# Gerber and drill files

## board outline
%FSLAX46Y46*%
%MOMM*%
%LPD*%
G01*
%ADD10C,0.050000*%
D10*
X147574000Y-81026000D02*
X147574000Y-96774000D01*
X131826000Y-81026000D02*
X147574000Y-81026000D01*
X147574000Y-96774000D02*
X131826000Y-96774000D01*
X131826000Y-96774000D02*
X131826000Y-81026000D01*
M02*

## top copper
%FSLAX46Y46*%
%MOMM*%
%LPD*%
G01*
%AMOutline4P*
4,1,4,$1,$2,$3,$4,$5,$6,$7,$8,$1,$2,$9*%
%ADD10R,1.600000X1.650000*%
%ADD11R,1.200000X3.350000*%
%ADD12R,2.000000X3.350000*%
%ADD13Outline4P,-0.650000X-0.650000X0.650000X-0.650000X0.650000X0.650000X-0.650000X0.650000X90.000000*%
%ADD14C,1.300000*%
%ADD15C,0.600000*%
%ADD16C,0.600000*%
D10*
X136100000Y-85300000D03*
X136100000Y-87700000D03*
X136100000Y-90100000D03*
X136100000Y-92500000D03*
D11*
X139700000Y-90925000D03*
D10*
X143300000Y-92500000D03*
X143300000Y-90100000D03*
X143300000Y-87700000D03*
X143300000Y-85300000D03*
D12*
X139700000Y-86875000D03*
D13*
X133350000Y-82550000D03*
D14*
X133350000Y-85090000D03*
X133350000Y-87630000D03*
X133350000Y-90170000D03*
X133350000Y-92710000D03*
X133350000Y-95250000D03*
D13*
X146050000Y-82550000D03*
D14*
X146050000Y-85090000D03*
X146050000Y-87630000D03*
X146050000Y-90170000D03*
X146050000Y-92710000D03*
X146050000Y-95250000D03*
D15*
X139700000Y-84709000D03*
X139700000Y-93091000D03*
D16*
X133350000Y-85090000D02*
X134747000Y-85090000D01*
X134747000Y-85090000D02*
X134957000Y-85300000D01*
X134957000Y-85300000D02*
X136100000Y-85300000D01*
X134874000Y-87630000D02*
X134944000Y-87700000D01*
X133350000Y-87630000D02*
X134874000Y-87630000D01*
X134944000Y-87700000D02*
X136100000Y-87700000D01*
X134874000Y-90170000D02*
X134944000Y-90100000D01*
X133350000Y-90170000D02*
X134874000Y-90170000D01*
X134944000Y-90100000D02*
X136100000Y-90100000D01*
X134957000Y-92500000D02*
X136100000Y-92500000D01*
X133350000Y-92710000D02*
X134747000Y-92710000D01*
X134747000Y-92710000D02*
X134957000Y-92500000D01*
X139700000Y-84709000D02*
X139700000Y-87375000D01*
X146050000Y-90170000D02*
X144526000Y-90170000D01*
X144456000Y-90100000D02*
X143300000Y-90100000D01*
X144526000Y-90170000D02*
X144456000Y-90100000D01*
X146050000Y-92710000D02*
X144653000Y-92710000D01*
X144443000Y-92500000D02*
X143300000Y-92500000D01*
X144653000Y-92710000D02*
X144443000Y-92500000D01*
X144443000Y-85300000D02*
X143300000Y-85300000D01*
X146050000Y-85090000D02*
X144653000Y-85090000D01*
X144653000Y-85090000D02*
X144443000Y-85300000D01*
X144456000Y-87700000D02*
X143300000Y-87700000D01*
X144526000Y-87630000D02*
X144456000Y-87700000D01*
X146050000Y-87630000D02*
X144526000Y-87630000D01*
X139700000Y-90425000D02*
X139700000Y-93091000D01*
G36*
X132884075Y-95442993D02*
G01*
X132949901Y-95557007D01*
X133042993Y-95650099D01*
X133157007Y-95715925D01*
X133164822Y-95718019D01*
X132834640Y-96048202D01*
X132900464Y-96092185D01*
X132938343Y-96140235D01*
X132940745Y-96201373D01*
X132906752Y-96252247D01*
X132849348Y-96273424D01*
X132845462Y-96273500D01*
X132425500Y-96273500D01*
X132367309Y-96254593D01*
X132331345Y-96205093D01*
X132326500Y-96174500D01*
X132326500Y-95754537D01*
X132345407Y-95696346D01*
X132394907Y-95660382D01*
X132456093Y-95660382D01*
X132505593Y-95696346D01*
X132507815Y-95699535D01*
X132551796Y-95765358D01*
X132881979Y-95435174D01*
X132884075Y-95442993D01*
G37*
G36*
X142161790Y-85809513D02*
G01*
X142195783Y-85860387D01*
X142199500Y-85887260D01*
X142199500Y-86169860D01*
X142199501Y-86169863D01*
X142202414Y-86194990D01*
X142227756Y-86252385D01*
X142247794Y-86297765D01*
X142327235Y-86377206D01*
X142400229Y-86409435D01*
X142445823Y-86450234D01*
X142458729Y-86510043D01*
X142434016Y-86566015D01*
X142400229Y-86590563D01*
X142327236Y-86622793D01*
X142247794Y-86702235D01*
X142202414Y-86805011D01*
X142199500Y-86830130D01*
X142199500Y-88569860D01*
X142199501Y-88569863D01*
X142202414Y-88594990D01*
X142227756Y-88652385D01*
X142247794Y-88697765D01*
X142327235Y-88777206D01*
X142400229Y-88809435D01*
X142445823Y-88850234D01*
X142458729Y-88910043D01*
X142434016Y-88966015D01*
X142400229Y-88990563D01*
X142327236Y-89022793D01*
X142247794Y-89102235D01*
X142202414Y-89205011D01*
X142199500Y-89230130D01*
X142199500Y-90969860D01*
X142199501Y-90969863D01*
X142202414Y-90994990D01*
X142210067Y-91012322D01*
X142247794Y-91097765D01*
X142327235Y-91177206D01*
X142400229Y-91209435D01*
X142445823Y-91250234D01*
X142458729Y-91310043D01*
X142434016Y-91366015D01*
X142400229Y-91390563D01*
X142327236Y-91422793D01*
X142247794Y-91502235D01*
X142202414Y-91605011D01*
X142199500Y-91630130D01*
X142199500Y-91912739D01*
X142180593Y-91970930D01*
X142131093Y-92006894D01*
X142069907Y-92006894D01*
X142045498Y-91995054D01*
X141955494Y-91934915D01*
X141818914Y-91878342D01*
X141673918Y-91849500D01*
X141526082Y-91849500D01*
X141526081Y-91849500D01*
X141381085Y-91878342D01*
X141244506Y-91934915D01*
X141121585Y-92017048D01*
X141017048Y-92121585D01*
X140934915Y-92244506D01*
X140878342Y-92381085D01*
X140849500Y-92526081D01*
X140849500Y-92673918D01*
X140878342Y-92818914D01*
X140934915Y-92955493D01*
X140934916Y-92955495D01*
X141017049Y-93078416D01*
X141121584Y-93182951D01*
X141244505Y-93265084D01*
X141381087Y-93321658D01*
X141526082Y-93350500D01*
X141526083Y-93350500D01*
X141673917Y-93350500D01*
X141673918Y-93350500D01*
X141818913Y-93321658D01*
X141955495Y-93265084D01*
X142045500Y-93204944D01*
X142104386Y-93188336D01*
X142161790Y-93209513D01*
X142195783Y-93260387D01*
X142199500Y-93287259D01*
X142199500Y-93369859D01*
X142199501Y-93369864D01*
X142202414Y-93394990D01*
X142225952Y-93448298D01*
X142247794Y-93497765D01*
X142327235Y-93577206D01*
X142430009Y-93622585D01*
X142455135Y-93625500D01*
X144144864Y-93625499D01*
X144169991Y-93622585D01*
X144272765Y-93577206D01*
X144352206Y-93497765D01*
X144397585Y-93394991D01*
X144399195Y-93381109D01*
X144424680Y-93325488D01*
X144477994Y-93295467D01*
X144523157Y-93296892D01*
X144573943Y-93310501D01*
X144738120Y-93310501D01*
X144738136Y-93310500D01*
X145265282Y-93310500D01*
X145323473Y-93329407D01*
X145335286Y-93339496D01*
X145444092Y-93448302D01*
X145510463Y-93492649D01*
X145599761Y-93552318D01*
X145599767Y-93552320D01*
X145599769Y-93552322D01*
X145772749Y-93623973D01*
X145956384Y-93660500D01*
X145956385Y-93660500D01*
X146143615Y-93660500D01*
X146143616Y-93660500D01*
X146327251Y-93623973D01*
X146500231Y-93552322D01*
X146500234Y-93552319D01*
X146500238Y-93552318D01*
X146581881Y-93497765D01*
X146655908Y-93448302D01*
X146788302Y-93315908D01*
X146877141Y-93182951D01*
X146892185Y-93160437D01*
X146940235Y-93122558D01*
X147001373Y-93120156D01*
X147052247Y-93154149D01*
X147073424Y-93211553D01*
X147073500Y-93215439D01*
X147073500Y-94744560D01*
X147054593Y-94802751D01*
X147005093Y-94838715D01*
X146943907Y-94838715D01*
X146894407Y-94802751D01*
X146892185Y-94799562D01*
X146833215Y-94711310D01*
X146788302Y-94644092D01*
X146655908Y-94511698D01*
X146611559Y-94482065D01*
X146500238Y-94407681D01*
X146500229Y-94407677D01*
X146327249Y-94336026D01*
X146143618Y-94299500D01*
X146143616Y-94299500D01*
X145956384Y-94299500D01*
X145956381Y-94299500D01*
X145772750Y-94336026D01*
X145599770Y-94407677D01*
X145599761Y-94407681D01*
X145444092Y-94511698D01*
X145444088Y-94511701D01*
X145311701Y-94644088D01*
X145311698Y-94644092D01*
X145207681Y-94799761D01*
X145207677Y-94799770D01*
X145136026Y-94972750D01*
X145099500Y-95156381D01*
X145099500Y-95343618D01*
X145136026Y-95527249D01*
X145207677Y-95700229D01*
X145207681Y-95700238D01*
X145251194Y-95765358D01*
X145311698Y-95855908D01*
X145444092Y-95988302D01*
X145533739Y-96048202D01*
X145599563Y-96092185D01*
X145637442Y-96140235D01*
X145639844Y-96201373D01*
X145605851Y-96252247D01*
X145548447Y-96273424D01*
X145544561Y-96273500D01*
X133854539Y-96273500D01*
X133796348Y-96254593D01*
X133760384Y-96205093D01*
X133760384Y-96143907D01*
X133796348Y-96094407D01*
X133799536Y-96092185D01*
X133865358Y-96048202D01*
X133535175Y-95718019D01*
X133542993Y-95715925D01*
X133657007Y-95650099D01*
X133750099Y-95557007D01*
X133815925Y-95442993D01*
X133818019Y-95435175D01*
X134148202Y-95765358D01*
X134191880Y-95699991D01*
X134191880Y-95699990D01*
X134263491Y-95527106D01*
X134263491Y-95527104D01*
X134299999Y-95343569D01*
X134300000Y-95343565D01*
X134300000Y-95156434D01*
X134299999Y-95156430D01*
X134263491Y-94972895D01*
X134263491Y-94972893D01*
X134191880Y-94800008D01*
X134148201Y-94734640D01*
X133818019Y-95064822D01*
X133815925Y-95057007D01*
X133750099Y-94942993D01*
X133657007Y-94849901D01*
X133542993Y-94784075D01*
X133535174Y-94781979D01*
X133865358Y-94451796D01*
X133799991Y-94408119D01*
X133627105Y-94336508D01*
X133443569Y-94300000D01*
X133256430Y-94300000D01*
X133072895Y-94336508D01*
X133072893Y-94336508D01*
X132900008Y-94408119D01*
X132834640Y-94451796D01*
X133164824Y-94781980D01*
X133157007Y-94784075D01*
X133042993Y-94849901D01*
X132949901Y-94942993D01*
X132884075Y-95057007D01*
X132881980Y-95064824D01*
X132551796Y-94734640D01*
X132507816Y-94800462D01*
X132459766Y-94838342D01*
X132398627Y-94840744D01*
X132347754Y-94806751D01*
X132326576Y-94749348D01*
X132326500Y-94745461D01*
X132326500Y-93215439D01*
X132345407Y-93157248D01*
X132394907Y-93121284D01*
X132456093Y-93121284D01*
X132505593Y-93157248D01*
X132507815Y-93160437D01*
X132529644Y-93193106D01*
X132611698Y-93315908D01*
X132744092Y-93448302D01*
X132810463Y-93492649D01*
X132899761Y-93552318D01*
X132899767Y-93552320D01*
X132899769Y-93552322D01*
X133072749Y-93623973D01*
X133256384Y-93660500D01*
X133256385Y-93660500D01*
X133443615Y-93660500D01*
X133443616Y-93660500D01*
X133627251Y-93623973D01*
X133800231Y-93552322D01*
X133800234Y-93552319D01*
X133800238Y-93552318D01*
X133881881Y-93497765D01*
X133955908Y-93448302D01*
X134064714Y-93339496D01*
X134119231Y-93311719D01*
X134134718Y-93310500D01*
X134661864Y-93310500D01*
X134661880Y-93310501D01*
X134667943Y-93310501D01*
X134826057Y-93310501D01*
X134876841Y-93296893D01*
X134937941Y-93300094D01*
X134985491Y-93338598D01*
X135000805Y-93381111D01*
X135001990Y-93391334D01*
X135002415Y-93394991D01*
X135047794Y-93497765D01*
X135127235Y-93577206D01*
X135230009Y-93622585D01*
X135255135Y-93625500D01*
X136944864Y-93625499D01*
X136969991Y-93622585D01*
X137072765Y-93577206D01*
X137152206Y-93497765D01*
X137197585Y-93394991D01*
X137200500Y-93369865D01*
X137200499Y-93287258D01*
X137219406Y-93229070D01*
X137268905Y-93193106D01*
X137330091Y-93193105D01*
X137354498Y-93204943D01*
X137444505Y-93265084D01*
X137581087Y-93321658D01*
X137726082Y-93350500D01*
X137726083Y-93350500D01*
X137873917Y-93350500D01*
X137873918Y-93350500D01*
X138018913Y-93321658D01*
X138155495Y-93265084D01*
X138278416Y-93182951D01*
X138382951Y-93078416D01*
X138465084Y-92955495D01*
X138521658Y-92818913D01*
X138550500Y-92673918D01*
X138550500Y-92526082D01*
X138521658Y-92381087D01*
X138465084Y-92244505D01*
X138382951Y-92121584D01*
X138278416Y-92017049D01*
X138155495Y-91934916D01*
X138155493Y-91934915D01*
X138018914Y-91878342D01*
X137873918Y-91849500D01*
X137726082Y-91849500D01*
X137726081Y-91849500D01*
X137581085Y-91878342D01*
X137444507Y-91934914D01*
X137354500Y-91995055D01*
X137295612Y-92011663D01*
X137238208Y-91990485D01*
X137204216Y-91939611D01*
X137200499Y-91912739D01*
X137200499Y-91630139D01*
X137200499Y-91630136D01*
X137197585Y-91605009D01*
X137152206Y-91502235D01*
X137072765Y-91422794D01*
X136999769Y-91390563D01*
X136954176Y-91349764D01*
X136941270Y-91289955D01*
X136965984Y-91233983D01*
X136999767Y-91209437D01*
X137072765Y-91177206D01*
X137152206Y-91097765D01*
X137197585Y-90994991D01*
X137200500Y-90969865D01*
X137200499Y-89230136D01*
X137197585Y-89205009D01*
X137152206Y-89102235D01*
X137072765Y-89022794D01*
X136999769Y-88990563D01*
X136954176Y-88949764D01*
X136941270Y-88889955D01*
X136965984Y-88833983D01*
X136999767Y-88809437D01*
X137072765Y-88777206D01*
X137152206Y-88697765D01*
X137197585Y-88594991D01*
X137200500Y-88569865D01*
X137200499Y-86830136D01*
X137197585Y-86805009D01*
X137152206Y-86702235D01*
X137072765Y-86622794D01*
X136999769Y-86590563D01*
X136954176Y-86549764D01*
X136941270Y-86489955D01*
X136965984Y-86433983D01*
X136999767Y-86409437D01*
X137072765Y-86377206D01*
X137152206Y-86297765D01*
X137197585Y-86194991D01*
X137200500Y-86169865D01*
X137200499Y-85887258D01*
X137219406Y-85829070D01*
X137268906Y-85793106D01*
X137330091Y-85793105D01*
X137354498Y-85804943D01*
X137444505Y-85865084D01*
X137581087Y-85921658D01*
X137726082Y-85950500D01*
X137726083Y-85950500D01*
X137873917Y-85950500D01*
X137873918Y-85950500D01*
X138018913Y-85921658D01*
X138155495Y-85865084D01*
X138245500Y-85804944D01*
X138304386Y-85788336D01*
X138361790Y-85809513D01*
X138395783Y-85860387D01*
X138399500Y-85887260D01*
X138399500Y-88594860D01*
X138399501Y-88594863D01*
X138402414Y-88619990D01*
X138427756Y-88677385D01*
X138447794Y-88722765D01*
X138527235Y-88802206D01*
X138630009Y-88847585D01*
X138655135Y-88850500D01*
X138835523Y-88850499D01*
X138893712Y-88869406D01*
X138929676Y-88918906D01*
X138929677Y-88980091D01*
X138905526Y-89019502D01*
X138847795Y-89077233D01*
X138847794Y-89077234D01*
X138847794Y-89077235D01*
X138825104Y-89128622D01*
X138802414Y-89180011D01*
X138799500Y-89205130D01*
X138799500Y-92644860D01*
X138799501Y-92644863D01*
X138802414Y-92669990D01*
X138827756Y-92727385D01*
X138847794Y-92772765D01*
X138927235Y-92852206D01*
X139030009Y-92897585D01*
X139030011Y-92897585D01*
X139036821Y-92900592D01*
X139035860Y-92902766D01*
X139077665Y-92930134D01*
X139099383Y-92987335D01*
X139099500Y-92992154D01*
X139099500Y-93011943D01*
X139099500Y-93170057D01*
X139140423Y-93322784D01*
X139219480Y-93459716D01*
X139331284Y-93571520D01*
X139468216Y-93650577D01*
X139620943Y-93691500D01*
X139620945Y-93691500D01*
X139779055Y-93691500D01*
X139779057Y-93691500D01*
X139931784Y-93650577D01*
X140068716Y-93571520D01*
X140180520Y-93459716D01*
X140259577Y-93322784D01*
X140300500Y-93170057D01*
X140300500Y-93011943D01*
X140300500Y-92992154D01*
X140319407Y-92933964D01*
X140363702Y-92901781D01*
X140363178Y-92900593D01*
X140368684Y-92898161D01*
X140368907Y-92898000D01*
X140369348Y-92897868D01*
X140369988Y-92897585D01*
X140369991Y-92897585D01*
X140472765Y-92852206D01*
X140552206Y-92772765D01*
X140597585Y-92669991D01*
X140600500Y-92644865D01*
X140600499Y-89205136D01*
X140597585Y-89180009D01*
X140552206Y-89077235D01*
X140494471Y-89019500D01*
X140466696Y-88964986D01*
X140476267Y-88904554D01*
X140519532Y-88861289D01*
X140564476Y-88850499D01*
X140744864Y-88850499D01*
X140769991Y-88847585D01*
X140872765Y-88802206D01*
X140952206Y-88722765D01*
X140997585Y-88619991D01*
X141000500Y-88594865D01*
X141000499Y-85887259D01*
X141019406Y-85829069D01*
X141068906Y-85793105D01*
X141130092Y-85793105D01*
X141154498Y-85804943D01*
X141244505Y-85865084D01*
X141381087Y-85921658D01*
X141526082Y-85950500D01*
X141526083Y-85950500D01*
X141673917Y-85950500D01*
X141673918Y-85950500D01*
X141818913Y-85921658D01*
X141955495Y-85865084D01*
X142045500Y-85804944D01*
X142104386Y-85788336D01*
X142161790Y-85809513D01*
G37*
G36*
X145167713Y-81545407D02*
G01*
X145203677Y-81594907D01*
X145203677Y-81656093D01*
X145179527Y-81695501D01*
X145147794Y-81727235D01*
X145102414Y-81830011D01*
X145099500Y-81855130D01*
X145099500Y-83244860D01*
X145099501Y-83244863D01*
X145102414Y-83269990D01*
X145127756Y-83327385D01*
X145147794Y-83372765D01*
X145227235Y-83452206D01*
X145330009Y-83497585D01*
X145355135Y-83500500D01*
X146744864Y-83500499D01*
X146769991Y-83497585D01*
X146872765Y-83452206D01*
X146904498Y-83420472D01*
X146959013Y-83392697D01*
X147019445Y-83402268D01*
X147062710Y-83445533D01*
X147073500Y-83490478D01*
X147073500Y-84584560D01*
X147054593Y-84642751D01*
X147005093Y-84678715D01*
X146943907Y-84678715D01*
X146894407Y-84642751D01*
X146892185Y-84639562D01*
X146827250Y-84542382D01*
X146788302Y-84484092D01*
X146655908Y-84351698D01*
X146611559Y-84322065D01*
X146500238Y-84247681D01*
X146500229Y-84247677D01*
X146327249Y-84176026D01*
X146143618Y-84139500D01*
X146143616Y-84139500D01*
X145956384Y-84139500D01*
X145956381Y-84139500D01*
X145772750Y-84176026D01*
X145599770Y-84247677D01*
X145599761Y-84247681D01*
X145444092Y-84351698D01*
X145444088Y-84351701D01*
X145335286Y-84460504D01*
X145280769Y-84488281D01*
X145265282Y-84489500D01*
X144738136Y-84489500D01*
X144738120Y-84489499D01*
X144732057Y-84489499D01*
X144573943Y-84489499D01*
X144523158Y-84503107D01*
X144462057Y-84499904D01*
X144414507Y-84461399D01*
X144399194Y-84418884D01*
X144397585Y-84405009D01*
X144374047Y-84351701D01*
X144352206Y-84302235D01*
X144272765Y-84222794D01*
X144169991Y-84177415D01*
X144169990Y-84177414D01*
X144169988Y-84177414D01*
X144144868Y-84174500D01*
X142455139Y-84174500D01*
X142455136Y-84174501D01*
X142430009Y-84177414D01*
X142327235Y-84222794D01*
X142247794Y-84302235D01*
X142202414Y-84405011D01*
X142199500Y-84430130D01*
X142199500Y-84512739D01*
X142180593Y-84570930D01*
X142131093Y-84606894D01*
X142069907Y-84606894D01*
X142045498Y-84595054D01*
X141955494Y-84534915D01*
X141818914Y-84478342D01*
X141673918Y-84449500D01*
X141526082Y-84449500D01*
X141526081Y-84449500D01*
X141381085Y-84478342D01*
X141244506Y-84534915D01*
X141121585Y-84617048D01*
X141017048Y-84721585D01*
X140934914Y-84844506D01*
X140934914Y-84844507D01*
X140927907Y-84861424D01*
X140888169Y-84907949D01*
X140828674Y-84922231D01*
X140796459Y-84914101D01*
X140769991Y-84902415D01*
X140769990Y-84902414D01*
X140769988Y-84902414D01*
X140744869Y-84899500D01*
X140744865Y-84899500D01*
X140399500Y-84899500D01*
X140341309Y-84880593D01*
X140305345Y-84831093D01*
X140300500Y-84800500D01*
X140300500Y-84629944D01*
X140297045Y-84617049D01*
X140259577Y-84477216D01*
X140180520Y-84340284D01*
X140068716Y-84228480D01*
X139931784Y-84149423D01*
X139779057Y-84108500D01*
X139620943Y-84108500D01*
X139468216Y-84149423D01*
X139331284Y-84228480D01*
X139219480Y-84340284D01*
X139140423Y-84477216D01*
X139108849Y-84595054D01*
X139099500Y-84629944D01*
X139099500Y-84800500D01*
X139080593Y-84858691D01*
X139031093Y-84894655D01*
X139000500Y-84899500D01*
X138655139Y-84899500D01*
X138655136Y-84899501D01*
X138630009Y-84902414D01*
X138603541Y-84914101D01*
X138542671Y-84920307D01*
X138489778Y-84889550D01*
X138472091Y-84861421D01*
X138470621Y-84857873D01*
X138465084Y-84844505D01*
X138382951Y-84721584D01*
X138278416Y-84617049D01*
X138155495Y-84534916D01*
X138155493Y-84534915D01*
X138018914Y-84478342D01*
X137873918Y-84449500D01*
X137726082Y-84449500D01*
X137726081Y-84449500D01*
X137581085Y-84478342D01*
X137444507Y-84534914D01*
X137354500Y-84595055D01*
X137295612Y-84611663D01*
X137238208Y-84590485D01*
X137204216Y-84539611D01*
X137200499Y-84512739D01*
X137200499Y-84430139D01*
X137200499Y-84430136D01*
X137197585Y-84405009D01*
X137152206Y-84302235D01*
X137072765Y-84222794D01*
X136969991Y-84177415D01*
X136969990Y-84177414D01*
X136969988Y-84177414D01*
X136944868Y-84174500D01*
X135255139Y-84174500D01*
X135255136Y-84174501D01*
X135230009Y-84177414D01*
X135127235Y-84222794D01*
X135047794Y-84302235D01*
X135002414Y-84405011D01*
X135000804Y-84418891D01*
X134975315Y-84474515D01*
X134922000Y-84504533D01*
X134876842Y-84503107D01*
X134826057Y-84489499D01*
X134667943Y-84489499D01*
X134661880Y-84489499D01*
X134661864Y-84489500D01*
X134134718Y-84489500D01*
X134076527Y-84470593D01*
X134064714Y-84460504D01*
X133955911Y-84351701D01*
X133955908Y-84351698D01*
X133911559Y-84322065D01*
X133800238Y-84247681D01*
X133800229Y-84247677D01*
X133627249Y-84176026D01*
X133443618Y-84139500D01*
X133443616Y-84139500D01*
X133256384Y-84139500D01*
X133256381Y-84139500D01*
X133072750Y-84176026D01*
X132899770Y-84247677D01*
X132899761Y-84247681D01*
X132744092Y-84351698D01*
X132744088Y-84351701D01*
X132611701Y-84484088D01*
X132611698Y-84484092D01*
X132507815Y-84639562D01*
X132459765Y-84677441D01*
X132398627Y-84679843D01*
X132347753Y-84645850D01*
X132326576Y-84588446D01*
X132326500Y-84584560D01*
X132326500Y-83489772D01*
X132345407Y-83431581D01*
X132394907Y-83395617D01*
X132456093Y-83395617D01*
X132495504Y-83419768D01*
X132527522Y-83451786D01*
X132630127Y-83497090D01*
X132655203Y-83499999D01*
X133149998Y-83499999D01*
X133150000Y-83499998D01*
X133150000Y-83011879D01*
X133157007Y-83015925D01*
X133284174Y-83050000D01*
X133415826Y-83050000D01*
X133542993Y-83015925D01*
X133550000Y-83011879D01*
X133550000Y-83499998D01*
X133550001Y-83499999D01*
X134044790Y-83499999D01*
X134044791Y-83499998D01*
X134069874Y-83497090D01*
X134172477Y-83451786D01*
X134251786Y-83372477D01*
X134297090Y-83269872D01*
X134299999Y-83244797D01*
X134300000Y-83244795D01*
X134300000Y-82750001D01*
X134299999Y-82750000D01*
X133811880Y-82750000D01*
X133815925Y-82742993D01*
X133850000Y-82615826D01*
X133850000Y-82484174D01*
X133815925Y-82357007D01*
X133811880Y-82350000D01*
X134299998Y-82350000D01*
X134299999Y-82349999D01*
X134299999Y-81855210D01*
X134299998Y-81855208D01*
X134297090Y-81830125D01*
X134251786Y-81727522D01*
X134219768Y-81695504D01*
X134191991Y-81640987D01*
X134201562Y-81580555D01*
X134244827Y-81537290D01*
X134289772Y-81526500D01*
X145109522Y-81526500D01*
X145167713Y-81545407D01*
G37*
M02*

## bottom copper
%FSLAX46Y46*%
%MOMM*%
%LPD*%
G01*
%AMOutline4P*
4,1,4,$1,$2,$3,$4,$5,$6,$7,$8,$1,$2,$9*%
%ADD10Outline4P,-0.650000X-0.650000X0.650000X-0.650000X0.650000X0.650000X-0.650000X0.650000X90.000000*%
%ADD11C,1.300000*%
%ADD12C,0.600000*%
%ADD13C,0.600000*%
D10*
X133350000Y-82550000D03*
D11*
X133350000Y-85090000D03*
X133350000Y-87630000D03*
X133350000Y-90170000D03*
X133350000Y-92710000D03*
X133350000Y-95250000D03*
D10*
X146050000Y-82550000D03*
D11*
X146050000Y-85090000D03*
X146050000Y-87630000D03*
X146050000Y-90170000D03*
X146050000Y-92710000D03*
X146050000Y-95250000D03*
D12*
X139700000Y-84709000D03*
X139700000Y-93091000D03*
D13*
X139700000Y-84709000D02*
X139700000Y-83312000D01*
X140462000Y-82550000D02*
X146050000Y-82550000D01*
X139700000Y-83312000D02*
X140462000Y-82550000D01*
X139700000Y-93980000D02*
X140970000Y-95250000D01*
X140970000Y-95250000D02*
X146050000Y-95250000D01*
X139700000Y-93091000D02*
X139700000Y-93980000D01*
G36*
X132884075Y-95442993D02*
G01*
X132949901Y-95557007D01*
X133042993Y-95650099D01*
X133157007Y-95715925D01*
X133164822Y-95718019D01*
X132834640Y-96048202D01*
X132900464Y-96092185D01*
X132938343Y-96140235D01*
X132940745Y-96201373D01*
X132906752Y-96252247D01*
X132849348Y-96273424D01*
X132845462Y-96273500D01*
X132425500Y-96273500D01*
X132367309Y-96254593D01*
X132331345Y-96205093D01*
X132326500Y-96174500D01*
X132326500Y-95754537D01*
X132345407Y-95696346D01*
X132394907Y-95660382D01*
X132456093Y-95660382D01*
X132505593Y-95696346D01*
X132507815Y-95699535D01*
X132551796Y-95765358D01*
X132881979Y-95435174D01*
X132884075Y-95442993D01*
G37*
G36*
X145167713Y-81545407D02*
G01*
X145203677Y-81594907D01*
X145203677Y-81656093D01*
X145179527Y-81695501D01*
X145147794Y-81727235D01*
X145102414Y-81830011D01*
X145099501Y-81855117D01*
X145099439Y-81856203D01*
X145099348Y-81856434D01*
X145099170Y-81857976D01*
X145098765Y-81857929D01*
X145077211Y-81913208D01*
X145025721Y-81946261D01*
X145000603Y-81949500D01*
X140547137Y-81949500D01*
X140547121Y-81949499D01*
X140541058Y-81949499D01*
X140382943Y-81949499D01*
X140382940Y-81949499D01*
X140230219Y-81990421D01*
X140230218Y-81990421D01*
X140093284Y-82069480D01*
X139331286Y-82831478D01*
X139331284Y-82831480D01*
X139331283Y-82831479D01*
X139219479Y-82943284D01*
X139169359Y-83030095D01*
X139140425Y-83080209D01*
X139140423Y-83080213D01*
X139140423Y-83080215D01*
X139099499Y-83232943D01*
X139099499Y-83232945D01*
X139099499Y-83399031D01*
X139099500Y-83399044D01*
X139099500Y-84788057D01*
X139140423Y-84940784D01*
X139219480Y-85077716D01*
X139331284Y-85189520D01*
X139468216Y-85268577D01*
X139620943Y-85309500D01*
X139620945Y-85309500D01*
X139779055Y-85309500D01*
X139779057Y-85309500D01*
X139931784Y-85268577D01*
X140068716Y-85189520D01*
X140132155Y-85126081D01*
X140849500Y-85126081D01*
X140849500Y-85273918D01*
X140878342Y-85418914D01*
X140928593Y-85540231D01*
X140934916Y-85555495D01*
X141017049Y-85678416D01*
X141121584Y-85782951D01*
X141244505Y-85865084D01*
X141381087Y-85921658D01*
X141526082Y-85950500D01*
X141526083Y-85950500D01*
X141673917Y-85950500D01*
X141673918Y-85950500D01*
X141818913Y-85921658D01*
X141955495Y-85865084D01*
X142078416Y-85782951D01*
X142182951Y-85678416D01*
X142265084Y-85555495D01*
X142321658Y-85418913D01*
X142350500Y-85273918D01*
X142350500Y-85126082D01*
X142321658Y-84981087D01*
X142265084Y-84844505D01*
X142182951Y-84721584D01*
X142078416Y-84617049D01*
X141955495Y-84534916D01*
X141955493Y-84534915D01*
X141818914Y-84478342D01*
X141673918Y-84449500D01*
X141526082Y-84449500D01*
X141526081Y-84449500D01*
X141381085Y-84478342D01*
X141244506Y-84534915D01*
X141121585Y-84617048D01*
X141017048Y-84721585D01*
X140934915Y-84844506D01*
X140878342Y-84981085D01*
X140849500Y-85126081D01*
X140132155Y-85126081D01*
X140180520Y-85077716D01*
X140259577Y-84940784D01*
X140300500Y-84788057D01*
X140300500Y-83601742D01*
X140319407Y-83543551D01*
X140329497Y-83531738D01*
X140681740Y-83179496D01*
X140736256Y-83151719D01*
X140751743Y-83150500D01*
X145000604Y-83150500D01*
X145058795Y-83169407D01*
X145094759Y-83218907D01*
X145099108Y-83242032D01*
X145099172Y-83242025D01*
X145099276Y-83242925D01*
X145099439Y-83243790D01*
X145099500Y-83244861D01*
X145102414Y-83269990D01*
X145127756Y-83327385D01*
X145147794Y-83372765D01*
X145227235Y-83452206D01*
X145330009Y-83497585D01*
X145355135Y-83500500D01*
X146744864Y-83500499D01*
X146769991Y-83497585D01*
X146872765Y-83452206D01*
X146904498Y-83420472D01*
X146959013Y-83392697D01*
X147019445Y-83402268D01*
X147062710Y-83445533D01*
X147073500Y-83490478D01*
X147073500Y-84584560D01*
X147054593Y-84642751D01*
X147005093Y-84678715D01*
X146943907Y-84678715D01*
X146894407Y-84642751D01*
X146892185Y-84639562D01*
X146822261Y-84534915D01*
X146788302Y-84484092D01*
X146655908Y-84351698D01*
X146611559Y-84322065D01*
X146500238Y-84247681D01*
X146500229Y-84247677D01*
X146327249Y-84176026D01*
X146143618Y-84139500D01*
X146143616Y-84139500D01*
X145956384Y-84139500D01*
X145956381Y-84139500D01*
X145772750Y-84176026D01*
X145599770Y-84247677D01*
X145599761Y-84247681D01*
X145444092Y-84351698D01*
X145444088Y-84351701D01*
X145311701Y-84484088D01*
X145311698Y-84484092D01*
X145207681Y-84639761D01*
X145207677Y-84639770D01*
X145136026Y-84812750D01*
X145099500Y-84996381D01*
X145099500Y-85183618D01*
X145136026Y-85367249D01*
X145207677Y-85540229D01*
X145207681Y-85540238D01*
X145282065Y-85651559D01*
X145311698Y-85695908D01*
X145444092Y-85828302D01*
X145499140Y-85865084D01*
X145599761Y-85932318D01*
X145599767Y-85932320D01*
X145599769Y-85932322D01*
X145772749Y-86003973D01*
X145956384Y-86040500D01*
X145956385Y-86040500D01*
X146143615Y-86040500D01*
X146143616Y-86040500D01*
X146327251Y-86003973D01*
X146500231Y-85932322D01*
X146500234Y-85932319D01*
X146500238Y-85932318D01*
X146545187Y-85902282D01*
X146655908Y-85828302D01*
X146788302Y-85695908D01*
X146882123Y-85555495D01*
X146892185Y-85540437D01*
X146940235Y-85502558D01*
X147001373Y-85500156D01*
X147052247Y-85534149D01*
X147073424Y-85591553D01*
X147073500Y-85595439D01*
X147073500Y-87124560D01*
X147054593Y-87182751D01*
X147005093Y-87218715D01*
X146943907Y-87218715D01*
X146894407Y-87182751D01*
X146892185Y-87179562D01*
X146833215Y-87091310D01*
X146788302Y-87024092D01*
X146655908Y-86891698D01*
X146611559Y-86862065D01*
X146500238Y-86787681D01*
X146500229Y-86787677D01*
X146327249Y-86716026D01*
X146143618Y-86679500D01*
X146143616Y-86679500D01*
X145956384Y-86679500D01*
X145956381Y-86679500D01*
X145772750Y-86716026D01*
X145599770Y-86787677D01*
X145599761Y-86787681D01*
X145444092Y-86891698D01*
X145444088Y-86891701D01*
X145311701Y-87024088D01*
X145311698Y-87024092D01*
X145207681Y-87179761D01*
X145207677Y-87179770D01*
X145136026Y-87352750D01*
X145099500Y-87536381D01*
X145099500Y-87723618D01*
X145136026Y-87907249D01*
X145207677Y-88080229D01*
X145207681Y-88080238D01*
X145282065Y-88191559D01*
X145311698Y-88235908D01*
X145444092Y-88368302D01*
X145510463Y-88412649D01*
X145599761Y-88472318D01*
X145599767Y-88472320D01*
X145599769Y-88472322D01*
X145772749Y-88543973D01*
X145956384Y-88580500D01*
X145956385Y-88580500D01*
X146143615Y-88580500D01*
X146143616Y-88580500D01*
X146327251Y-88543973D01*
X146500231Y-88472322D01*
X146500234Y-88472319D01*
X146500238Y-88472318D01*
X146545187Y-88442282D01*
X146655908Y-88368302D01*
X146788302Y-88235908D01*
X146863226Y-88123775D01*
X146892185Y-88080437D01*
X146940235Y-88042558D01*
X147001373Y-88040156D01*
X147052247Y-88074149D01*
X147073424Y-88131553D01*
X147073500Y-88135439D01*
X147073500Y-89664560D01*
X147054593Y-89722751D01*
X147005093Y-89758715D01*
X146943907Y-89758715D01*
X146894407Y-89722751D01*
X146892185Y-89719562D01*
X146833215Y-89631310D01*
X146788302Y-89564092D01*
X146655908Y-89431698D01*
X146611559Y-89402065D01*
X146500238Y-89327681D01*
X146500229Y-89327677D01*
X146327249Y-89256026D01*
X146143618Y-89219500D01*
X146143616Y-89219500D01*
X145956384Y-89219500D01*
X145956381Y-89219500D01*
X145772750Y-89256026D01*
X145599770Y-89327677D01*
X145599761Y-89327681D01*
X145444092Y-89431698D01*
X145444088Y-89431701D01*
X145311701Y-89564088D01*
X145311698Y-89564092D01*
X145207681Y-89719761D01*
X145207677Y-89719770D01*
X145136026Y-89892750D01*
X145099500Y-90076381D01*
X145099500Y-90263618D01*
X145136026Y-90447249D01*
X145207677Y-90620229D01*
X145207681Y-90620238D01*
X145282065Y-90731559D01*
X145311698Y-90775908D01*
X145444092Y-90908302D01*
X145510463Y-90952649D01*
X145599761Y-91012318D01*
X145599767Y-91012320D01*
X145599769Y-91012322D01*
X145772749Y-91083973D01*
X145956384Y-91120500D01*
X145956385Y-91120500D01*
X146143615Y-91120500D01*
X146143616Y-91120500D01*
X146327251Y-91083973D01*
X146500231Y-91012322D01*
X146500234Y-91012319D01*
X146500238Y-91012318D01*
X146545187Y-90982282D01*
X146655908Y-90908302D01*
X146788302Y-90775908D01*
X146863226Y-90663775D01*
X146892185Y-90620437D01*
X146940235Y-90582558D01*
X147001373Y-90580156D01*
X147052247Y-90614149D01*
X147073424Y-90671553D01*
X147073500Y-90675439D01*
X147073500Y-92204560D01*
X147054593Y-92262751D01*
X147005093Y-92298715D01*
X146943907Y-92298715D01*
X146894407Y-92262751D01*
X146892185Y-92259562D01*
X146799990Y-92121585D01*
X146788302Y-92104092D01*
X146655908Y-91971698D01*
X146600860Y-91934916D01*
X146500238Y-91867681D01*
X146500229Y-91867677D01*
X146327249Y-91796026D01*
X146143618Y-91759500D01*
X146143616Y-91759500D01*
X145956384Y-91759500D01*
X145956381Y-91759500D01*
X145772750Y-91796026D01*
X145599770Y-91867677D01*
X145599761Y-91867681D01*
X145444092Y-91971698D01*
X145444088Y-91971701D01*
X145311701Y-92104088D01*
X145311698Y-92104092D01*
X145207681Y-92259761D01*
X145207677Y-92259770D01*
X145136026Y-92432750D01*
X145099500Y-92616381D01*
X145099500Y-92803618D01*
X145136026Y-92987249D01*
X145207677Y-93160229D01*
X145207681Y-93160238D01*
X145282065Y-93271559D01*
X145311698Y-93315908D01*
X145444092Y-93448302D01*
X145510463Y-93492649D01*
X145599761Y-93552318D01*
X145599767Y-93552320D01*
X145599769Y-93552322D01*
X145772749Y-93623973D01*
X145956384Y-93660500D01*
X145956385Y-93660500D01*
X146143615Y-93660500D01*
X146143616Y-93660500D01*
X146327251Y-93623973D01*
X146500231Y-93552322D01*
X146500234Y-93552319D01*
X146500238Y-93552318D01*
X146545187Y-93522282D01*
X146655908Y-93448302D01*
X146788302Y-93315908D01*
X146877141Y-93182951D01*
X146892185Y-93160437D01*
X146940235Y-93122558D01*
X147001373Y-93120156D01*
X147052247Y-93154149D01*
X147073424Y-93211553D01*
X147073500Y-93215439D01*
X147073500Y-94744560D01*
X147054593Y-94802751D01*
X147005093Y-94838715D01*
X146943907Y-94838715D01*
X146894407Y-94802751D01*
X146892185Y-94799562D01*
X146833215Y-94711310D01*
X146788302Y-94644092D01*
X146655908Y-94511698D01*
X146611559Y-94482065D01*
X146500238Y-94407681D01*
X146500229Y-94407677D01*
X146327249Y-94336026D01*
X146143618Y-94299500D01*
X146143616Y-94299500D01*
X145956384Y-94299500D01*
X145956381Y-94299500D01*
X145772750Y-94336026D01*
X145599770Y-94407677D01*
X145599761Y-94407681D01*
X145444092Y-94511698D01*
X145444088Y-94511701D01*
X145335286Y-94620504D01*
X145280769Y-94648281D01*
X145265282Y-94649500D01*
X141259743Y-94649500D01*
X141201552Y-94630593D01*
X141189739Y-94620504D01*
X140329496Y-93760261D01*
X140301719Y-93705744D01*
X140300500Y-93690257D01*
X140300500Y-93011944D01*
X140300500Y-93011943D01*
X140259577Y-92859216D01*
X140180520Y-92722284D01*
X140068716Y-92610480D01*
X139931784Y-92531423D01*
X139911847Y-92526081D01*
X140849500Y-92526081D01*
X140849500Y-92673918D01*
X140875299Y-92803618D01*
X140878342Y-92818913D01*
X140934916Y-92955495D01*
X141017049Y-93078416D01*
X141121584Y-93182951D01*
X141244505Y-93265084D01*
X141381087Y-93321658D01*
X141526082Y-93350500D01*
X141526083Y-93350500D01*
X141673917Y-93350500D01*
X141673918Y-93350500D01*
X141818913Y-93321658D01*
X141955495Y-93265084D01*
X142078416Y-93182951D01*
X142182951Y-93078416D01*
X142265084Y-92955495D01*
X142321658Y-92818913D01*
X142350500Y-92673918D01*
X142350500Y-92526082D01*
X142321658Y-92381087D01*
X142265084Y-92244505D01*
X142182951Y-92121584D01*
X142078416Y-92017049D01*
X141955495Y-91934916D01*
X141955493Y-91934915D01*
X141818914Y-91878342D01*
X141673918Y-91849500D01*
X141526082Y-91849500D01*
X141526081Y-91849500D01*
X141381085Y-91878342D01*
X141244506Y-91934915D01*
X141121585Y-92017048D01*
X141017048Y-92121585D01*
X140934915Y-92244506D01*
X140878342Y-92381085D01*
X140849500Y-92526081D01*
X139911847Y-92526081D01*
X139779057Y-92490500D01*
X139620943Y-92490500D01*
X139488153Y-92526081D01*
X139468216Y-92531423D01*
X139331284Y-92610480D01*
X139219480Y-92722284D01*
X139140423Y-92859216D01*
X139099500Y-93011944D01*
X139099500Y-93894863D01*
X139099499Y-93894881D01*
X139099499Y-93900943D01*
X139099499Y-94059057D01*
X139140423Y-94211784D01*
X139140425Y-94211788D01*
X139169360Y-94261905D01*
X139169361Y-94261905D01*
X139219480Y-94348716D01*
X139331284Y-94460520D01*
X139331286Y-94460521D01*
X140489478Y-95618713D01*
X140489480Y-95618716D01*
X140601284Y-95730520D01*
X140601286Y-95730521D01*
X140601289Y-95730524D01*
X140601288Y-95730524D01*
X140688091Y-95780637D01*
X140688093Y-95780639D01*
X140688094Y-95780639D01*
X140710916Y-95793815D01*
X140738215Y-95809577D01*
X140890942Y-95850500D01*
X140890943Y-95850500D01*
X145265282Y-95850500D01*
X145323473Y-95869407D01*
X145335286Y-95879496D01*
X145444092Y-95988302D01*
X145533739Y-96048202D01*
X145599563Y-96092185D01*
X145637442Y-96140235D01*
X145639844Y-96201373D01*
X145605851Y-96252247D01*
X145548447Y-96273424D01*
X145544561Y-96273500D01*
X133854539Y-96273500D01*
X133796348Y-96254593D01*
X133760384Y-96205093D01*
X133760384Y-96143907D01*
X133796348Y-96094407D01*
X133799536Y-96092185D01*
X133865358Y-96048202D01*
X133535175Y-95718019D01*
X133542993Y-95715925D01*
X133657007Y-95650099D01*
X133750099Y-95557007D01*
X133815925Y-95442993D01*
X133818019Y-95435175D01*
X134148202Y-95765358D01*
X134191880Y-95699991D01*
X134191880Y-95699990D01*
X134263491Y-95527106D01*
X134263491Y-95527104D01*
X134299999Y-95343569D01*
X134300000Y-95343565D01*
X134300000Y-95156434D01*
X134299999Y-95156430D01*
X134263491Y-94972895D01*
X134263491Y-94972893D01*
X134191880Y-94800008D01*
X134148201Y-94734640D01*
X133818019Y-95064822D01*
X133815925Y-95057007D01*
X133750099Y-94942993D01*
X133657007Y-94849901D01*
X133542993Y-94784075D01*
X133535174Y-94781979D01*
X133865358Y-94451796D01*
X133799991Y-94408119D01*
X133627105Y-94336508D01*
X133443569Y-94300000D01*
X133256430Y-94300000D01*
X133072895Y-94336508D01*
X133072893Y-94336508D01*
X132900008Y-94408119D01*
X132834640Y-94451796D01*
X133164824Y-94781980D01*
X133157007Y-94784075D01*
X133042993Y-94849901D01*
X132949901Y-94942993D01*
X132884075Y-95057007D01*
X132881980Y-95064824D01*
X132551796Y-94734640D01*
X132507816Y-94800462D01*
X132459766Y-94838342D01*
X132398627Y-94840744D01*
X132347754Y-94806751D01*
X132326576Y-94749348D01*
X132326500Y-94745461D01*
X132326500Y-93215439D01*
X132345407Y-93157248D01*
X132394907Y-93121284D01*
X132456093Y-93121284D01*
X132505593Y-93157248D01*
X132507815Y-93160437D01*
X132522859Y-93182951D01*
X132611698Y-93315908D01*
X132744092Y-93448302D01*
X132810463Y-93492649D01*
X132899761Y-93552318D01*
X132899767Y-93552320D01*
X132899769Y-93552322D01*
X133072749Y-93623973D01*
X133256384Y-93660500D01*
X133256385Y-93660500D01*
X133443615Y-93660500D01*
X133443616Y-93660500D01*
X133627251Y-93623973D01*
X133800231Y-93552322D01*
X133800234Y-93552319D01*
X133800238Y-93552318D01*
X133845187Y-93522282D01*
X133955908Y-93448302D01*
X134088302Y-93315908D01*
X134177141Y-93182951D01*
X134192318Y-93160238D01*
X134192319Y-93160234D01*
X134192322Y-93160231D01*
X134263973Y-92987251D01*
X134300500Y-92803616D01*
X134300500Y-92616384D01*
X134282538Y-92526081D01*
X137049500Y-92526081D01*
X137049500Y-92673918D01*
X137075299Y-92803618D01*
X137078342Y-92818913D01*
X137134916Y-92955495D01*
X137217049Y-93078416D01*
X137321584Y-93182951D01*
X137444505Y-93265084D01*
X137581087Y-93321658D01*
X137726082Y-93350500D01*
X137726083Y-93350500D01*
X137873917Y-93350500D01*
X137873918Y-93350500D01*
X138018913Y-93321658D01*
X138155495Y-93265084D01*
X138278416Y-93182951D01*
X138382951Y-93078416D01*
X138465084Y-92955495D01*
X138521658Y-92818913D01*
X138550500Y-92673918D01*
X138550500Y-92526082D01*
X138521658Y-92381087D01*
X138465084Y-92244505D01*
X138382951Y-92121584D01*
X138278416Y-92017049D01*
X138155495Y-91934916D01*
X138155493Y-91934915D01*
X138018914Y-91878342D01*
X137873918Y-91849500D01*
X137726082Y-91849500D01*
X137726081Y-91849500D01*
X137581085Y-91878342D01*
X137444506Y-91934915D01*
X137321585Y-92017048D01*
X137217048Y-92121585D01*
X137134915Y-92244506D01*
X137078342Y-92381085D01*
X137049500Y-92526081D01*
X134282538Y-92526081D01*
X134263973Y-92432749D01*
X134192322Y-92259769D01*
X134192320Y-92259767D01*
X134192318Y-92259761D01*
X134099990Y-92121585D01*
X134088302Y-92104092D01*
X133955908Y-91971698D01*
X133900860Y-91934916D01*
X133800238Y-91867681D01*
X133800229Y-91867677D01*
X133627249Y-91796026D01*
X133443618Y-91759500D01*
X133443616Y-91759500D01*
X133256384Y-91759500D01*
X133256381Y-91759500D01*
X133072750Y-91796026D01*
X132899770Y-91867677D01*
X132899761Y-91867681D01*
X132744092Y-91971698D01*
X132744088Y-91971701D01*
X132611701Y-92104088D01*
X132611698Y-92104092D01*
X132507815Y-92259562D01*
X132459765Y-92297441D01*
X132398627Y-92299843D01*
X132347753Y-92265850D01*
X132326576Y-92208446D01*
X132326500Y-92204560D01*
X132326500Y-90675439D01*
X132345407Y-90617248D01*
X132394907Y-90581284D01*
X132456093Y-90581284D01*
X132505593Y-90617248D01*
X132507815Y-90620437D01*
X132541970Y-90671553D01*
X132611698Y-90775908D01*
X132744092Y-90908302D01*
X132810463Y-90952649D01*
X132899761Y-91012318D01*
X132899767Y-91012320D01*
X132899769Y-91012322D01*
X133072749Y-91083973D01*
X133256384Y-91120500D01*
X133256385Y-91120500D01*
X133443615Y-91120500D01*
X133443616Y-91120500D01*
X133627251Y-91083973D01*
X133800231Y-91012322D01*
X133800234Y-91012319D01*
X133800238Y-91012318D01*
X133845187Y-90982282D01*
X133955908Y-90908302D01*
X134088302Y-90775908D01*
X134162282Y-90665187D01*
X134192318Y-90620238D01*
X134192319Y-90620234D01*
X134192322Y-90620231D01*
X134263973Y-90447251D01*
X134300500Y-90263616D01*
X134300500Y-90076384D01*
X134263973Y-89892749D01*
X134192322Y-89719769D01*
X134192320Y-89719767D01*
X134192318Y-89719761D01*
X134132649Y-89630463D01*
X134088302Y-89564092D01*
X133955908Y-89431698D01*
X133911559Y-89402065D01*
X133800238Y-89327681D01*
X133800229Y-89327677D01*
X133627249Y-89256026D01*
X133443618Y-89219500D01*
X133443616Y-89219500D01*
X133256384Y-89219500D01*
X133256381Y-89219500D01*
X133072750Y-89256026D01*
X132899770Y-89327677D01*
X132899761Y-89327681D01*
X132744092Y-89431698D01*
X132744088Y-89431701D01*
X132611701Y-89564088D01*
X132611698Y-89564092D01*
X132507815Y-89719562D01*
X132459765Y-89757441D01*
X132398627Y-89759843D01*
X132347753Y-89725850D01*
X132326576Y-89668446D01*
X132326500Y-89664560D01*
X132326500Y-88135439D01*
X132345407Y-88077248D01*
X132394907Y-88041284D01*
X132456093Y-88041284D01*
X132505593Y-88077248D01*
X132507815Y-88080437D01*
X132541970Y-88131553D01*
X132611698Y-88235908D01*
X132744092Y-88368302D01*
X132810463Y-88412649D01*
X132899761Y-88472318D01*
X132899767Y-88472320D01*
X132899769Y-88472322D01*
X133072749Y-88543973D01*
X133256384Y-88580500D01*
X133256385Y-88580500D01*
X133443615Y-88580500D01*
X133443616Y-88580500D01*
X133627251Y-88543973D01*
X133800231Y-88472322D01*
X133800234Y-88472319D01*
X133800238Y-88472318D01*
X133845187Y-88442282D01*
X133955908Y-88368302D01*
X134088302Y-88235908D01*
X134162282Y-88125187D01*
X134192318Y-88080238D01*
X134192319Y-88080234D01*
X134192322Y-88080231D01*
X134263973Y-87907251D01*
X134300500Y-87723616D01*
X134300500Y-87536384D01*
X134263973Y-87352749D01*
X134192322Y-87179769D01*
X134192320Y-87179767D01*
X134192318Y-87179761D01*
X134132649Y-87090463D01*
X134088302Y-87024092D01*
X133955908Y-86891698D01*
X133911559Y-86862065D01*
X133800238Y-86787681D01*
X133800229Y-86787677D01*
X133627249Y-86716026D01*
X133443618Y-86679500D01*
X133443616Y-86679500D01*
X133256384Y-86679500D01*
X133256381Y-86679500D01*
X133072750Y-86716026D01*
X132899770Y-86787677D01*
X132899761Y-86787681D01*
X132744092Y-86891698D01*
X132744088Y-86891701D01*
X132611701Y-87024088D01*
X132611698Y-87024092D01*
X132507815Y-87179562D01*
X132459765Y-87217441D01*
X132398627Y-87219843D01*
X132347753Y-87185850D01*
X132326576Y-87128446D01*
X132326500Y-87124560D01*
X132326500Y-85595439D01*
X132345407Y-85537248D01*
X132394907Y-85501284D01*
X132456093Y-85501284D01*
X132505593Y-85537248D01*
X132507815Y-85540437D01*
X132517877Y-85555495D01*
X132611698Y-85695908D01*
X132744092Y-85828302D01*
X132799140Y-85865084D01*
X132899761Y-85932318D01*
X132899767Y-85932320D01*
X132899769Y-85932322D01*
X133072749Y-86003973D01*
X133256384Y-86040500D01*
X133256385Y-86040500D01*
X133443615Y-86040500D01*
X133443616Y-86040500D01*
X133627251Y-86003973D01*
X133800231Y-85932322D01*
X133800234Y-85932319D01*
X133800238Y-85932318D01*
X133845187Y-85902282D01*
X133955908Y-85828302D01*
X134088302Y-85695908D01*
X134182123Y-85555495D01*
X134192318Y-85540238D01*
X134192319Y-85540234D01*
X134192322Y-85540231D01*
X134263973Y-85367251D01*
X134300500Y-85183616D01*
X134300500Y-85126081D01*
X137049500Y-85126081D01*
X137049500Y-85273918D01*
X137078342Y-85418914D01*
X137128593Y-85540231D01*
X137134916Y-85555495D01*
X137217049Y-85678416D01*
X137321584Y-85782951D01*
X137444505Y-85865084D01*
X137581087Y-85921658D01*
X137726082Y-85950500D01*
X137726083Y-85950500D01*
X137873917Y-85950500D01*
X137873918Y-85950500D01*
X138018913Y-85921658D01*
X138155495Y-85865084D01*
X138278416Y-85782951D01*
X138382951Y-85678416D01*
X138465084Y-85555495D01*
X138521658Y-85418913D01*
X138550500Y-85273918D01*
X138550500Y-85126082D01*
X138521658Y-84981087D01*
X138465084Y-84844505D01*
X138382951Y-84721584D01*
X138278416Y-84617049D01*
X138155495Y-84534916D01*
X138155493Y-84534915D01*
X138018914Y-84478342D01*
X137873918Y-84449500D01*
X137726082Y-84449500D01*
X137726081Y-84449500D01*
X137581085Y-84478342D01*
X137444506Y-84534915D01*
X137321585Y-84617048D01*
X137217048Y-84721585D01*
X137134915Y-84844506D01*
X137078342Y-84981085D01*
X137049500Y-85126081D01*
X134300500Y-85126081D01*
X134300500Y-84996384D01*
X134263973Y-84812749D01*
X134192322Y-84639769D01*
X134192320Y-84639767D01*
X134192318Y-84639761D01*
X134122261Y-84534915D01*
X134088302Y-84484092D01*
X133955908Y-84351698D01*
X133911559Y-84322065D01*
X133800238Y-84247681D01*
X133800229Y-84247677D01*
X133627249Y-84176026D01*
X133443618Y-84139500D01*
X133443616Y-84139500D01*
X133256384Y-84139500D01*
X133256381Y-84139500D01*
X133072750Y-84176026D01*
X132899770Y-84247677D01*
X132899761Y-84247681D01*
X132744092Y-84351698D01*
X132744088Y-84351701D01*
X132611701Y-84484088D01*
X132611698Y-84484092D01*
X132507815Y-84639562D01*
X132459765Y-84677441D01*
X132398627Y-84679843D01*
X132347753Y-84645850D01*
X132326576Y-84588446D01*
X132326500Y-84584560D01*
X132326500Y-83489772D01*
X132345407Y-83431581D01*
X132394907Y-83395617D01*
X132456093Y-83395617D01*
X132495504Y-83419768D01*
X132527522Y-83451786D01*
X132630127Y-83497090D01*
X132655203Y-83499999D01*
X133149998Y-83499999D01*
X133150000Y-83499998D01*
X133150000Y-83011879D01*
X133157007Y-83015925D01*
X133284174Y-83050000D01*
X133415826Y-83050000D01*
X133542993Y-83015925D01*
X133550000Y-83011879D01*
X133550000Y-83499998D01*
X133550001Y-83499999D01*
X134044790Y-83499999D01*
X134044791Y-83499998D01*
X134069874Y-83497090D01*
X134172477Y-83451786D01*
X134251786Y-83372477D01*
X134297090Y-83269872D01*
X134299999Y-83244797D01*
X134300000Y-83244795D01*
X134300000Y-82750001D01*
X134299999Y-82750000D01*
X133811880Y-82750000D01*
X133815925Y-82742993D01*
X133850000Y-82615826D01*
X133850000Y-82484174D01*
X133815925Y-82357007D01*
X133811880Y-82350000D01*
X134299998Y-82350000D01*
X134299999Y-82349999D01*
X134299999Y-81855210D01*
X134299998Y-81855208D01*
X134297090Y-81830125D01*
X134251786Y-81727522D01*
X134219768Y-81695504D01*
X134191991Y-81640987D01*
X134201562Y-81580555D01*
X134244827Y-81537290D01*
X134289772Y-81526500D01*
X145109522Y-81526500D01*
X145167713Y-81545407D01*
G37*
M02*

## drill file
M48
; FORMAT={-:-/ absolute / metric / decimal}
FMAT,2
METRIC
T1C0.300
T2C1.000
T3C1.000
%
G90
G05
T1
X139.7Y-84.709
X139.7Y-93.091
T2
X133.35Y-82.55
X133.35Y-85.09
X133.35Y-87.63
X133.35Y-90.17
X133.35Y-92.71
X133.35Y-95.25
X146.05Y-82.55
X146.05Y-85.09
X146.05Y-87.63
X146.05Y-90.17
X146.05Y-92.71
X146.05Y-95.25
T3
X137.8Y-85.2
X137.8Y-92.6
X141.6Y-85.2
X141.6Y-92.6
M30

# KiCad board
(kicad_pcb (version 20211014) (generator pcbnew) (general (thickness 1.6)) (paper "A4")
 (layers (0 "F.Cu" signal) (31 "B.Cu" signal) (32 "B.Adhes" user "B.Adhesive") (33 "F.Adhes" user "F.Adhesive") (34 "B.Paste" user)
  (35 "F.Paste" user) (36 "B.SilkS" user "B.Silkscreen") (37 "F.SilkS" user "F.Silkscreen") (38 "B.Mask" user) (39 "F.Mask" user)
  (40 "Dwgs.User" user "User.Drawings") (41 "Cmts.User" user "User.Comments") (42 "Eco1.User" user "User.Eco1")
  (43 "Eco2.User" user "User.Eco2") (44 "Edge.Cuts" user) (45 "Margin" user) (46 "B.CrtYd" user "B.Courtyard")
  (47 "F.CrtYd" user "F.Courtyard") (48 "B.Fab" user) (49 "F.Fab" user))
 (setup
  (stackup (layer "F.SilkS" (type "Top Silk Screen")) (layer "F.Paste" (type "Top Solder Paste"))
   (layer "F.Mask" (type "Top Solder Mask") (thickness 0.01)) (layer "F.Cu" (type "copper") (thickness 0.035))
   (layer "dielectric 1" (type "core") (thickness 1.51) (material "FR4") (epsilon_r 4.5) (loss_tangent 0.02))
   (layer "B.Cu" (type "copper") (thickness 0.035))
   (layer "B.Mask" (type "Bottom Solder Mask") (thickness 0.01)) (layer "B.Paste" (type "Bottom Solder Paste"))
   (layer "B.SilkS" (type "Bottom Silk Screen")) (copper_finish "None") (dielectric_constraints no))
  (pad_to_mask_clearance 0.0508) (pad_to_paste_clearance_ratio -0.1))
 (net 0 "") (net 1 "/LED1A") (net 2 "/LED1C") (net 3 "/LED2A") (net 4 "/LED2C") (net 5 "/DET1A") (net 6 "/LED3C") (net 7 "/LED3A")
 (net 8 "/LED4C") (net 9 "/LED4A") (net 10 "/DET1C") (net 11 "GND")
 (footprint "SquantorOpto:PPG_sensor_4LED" (layer "F.Cu") (at 139.7 88.9)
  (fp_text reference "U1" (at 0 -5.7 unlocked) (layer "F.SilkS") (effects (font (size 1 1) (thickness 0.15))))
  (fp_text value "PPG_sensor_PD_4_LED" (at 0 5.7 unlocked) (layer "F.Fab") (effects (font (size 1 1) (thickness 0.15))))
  (pad "" np_thru_hole circle (at -1.9 3.7) (size 1 1) (drill 1) (layers F&B.Cu *.Mask))
  (pad "" np_thru_hole circle (at 1.9 3.7) (size 1 1) (drill 1) (layers F&B.Cu *.Mask))
  (pad "" np_thru_hole circle (at -1.9 -3.7) (size 1 1) (drill 1) (layers F&B.Cu *.Mask))
  (pad "" np_thru_hole circle (at 1.9 -3.7) (size 1 1) (drill 1) (layers F&B.Cu *.Mask))
  (pad "1" smd rect (at -3.6 -3.6) (size 1.6 1.65) (layers "F.Cu" "F.Paste" "F.Mask") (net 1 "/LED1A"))
  (pad "2" smd rect (at -3.6 -1.2) (size 1.6 1.65) (layers "F.Cu" "F.Paste" "F.Mask") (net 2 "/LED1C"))
  (pad "3" smd rect (at -3.6 1.2) (size 1.6 1.65) (layers "F.Cu" "F.Paste" "F.Mask") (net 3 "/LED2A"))
  (pad "4" smd rect (at -3.6 3.6) (size 1.6 1.65) (layers "F.Cu" "F.Paste" "F.Mask") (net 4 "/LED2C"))
  (pad "5" smd rect (at 0 2.025) (size 1.2 3.35) (layers "F.Cu" "F.Paste" "F.Mask") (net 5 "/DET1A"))
  (pad "6" smd rect (at 3.6 3.6) (size 1.6 1.65) (layers "F.Cu" "F.Paste" "F.Mask") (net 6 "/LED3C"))
  (pad "7" smd rect (at 3.6 1.2) (size 1.6 1.65) (layers "F.Cu" "F.Paste" "F.Mask") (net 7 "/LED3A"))
  (pad "8" smd rect (at 3.6 -1.2) (size 1.6 1.65) (layers "F.Cu" "F.Paste" "F.Mask") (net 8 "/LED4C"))
  (pad "9" smd rect (at 3.6 -3.6) (size 1.6 1.65) (layers "F.Cu" "F.Paste" "F.Mask") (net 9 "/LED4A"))
  (pad "10" smd rect (at 0 -2.025) (size 2 3.35) (layers "F.Cu" "F.Paste" "F.Mask") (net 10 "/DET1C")))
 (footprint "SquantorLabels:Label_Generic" (layer "B.Cu") (at 139.7 93.7675 180)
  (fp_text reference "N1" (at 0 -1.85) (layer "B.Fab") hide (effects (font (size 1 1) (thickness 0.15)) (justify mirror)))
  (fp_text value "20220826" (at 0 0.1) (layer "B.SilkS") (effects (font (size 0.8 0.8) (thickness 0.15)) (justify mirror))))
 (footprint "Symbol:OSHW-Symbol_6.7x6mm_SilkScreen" (layer "B.Cu") (at 139.7 88.646 180)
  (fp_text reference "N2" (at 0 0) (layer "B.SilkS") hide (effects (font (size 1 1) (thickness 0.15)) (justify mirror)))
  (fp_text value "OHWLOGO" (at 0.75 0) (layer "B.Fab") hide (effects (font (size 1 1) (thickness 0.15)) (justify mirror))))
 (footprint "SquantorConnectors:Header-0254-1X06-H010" (layer "B.Cu") (at 133.35 88.9 -90)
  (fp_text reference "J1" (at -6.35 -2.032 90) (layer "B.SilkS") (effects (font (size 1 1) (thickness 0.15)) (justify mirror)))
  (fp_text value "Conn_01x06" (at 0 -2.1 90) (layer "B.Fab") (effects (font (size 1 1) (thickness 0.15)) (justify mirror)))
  (pad "1" thru_hole trapezoid locked (at -6.35 0 90) (size 1.3 1.3) (drill 1) (layers *.Cu *.Mask) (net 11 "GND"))
  (pad "2" thru_hole circle locked (at -3.81 0 90) (size 1.3 1.3) (drill 1) (layers *.Cu *.Mask) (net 1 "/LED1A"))
  (pad "3" thru_hole circle locked (at -1.27 0 90) (size 1.3 1.3) (drill 1) (layers *.Cu *.Mask) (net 2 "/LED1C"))
  (pad "4" thru_hole circle locked (at 1.27 0 90) (size 1.3 1.3) (drill 1) (layers *.Cu *.Mask) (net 3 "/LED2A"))
  (pad "5" thru_hole circle locked (at 3.81 0 90) (size 1.3 1.3) (drill 1) (layers *.Cu *.Mask) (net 4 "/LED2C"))
  (pad "6" thru_hole circle locked (at 6.35 0 90) (size 1.3 1.3) (drill 1) (layers *.Cu *.Mask) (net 11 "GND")))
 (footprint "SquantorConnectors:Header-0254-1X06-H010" (layer "B.Cu") (at 146.05 88.9 -90)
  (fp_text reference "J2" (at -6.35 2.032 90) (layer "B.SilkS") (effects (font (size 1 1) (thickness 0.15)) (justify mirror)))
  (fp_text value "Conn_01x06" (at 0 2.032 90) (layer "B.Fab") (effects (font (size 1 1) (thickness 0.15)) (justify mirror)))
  (pad "1" thru_hole trapezoid locked (at -6.35 0 90) (size 1.3 1.3) (drill 1) (layers *.Cu *.Mask) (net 10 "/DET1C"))
  (pad "2" thru_hole circle locked (at -3.81 0 90) (size 1.3 1.3) (drill 1) (layers *.Cu *.Mask) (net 9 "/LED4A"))
  (pad "3" thru_hole circle locked (at -1.27 0 90) (size 1.3 1.3) (drill 1) (layers *.Cu *.Mask) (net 8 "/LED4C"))
  (pad "4" thru_hole circle locked (at 1.27 0 90) (size 1.3 1.3) (drill 1) (layers *.Cu *.Mask) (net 7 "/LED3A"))
  (pad "5" thru_hole circle locked (at 3.81 0 90) (size 1.3 1.3) (drill 1) (layers *.Cu *.Mask) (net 6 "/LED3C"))
  (pad "6" thru_hole circle locked (at 6.35 0 90) (size 1.3 1.3) (drill 1) (layers *.Cu *.Mask) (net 5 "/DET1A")))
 (gr_line (start 147.574 81.026) (end 147.574 96.774) (layer "Edge.Cuts") (width 0.05))
 (gr_line (start 131.826 81.026) (end 147.574 81.026) (layer "Edge.Cuts") (width 0.05))
 (gr_line (start 147.574 96.774) (end 131.826 96.774) (layer "Edge.Cuts") (width 0.05))
 (gr_line (start 131.826 96.774) (end 131.826 81.026) (layer "Edge.Cuts") (width 0.05))
 (segment (start 133.35 85.09) (end 134.747 85.09) (width 0.6) (layer "F.Cu") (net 1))
 (segment (start 134.747 85.09) (end 134.957 85.3) (width 0.6) (layer "F.Cu") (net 1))
 (segment (start 134.957 85.3) (end 136.1 85.3) (width 0.6) (layer "F.Cu") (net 1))
 (segment (start 134.874 87.63) (end 134.944 87.7) (width 0.6) (layer "F.Cu") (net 2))
 (segment (start 133.35 87.63) (end 134.874 87.63) (width 0.6) (layer "F.Cu") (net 2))
 (segment (start 134.944 87.7) (end 136.1 87.7) (width 0.6) (layer "F.Cu") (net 2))
 (segment (start 134.874 90.17) (end 134.944 90.1) (width 0.6) (layer "F.Cu") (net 3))
 (segment (start 133.35 90.17) (end 134.874 90.17) (width 0.6) (layer "F.Cu") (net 3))
 (segment (start 134.944 90.1) (end 136.1 90.1) (width 0.6) (layer "F.Cu") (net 3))
 (segment (start 134.957 92.5) (end 136.1 92.5) (width 0.6) (layer "F.Cu") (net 4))
 (segment (start 133.35 92.71) (end 134.747 92.71) (width 0.6) (layer "F.Cu") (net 4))
 (segment (start 134.747 92.71) (end 134.957 92.5) (width 0.6) (layer "F.Cu") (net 4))
 (segment (start 139.7 84.709) (end 139.7 87.375) (width 0.6) (layer "F.Cu") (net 10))
 (via (at 139.7 84.709) (size 0.6) (drill 0.3) (layers "F.Cu" "B.Cu") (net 10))
 (segment (start 139.7 84.709) (end 139.7 83.312) (width 0.6) (layer "B.Cu") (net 10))
 (segment (start 140.462 82.55) (end 146.05 82.55) (width 0.6) (layer "B.Cu") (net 10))
 (segment (start 139.7 83.312) (end 140.462 82.55) (width 0.6) (layer "B.Cu") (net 10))
 (segment (start 146.05 90.17) (end 144.526 90.17) (width 0.6) (layer "F.Cu") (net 7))
 (segment (start 144.456 90.1) (end 143.3 90.1) (width 0.6) (layer "F.Cu") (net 7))
 (segment (start 144.526 90.17) (end 144.456 90.1) (width 0.6) (layer "F.Cu") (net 7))
 (segment (start 146.05 92.71) (end 144.653 92.71) (width 0.6) (layer "F.Cu") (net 6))
 (segment (start 144.443 92.5) (end 143.3 92.5) (width 0.6) (layer "F.Cu") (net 6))
 (segment (start 144.653 92.71) (end 144.443 92.5) (width 0.6) (layer "F.Cu") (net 6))
 (segment (start 144.443 85.3) (end 143.3 85.3) (width 0.6) (layer "F.Cu") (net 9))
 (segment (start 146.05 85.09) (end 144.653 85.09) (width 0.6) (layer "F.Cu") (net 9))
 (segment (start 144.653 85.09) (end 144.443 85.3) (width 0.6) (layer "F.Cu") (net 9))
 (segment (start 144.456 87.7) (end 143.3 87.7) (width 0.6) (layer "F.Cu") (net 8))
 (segment (start 144.526 87.63) (end 144.456 87.7) (width 0.6) (layer "F.Cu") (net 8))
 (segment (start 146.05 87.63) (end 144.526 87.63) (width 0.6) (layer "F.Cu") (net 8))
 (segment (start 139.7 90.425) (end 139.7 93.091) (width 0.6) (layer "F.Cu") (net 5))
 (via (at 139.7 93.091) (size 0.6) (drill 0.3) (layers "F.Cu" "B.Cu") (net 5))
 (segment (start 139.7 93.98) (end 140.97 95.25) (width 0.6) (layer "B.Cu") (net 5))
 (segment (start 140.97 95.25) (end 146.05 95.25) (width 0.6) (layer "B.Cu") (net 5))
 (segment (start 139.7 93.091) (end 139.7 93.98) (width 0.6) (layer "B.Cu") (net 5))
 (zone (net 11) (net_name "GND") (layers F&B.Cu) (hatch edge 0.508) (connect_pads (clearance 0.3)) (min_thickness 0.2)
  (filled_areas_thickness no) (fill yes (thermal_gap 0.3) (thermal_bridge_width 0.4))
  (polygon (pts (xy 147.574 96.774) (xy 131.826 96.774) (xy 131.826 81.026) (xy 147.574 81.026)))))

